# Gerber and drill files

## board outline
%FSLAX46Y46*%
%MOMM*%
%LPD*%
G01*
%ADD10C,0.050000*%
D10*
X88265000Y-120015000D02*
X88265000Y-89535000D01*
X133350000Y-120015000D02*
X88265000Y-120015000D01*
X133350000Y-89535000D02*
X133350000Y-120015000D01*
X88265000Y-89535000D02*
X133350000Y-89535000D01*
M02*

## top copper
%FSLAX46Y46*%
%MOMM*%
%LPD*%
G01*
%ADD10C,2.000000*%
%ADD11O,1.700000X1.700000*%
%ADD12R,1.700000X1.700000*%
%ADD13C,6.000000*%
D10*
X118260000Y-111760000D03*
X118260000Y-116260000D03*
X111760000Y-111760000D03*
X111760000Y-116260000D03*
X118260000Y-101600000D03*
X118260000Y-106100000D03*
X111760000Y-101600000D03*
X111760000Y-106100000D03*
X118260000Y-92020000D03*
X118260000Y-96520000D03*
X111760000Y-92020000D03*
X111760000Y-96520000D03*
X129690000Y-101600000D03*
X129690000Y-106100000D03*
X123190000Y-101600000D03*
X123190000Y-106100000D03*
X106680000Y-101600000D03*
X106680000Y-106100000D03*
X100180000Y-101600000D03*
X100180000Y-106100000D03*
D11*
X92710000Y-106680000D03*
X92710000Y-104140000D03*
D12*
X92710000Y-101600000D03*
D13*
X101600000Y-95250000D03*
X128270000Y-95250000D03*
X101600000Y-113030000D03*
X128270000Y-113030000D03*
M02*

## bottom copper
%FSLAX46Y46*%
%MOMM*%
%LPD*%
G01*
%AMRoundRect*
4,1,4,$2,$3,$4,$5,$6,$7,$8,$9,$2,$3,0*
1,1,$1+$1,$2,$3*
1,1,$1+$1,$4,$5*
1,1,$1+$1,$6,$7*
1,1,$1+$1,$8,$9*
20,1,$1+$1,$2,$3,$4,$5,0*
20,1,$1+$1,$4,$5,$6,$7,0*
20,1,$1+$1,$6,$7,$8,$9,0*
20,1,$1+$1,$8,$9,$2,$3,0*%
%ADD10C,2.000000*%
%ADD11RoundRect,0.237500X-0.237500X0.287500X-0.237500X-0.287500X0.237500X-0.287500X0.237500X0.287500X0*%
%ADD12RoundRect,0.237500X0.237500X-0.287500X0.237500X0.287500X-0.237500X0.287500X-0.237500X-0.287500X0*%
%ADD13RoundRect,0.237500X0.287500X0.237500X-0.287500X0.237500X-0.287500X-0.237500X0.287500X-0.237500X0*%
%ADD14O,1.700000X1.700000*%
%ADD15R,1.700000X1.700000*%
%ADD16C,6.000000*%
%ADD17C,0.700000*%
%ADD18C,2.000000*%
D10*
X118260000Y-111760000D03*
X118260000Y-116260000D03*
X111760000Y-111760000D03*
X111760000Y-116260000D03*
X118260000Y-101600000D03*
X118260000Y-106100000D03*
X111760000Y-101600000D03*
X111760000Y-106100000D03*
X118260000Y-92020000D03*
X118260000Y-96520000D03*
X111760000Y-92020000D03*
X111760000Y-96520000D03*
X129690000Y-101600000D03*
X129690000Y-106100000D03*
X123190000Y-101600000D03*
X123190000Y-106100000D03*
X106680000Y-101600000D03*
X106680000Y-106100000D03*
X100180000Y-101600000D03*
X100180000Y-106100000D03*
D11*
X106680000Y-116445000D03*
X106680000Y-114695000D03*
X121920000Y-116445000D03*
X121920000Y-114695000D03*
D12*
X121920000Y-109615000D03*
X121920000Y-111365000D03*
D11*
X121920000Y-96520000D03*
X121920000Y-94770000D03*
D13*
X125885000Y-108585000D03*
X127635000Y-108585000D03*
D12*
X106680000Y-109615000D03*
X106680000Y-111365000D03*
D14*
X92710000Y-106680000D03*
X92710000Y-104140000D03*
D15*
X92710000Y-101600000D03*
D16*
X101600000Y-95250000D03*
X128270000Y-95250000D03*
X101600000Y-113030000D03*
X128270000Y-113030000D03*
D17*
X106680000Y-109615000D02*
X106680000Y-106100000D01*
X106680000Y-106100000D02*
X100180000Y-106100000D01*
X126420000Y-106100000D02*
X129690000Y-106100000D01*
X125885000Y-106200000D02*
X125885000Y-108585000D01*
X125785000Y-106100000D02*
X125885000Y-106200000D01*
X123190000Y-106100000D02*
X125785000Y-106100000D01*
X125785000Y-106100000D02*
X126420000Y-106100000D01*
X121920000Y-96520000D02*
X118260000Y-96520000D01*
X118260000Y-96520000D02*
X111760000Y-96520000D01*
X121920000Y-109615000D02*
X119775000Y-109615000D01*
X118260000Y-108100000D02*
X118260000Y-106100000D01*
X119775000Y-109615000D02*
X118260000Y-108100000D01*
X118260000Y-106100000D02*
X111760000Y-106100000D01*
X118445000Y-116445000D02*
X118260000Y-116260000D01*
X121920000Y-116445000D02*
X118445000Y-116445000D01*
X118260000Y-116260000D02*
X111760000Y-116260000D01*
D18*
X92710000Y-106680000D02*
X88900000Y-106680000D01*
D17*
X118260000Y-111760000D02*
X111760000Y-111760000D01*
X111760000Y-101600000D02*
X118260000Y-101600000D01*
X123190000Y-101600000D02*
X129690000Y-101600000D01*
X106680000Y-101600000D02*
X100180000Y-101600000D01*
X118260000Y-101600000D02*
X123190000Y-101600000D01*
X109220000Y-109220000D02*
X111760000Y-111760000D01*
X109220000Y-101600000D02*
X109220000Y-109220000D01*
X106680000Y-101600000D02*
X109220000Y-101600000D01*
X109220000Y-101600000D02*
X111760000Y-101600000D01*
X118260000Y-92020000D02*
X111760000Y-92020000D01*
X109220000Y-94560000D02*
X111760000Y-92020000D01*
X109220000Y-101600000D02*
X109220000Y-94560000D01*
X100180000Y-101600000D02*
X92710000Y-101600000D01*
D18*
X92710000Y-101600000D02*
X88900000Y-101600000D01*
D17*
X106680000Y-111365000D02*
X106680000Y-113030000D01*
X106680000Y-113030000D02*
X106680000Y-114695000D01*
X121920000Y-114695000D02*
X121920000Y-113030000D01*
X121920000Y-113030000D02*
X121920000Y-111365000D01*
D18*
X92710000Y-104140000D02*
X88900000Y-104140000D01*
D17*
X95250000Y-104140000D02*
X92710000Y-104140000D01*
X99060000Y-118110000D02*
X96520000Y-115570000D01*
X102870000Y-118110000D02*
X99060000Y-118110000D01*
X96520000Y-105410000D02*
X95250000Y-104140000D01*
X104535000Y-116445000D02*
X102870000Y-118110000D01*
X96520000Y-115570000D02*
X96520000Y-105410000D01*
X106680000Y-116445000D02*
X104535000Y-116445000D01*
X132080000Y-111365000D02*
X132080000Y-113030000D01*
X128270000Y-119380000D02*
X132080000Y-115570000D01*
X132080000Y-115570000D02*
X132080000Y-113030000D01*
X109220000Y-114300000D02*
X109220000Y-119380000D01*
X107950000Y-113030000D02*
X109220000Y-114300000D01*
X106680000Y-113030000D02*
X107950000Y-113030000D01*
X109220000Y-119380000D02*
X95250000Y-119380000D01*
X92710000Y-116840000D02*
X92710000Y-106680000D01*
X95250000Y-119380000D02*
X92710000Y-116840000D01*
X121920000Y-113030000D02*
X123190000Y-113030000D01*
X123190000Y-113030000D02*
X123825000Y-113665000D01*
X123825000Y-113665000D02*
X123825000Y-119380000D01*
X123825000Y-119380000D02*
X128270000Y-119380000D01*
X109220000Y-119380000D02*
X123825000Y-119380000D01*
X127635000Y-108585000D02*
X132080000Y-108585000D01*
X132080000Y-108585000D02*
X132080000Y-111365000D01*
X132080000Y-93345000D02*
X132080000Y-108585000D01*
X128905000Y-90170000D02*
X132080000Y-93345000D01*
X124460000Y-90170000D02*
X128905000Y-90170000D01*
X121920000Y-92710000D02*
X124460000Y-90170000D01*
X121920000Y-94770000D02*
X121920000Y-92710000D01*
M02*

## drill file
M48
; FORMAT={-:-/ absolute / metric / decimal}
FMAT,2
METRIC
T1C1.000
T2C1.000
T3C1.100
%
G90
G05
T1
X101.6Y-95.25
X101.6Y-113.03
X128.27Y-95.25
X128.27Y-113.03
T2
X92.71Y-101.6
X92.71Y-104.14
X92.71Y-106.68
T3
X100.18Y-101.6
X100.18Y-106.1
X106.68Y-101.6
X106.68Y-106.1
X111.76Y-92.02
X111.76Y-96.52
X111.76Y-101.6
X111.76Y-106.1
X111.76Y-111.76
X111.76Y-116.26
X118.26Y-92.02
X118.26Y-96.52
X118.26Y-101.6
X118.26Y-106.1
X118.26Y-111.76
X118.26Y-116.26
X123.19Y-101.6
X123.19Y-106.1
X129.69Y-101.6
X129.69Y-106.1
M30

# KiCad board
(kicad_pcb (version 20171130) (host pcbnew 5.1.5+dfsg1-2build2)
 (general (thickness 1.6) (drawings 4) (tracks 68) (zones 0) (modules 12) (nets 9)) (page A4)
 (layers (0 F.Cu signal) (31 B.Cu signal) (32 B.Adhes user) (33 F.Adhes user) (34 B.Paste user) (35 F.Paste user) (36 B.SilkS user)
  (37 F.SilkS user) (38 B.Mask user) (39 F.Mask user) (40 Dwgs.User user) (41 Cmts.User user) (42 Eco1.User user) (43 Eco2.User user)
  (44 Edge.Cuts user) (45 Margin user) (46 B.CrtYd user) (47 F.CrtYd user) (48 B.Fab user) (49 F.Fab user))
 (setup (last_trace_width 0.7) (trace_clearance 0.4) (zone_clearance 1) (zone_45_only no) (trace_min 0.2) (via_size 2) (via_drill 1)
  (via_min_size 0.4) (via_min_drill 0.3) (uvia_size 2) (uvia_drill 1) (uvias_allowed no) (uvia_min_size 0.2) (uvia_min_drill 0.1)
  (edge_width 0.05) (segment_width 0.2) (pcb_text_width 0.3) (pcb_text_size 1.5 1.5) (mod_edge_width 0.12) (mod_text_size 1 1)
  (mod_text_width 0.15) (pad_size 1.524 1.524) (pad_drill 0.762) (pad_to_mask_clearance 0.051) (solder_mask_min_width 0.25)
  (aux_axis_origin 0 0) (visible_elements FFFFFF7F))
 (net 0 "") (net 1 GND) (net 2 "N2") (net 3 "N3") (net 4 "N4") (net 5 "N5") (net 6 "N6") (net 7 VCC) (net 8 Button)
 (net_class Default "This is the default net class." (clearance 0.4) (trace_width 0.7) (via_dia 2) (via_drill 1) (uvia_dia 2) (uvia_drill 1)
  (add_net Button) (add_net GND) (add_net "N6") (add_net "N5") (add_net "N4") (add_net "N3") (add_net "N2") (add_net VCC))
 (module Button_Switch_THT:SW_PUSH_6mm (layer F.Cu) (at 111.76 111.76)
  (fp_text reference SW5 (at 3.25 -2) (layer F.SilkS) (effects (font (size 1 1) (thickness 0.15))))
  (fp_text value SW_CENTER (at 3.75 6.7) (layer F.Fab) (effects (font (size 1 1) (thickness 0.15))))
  (pad 1 thru_hole circle (at 6.5 0 90) (size 2 2) (drill 1.1) (layers *.Cu *.Mask) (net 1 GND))
  (pad 2 thru_hole circle (at 6.5 4.5 90) (size 2 2) (drill 1.1) (layers *.Cu *.Mask) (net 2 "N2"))
  (pad 1 thru_hole circle (at 0 0 90) (size 2 2) (drill 1.1) (layers *.Cu *.Mask) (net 1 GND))
  (pad 2 thru_hole circle (at 0 4.5 90) (size 2 2) (drill 1.1) (layers *.Cu *.Mask) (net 2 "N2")))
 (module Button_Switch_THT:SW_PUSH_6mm (layer F.Cu) (at 111.76 101.6)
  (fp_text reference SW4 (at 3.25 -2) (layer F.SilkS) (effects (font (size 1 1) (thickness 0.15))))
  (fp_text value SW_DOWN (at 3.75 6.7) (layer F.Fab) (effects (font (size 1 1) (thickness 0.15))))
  (pad 1 thru_hole circle (at 6.5 0 90) (size 2 2) (drill 1.1) (layers *.Cu *.Mask) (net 1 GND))
  (pad 2 thru_hole circle (at 6.5 4.5 90) (size 2 2) (drill 1.1) (layers *.Cu *.Mask) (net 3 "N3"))
  (pad 1 thru_hole circle (at 0 0 90) (size 2 2) (drill 1.1) (layers *.Cu *.Mask) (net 1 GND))
  (pad 2 thru_hole circle (at 0 4.5 90) (size 2 2) (drill 1.1) (layers *.Cu *.Mask) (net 3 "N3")))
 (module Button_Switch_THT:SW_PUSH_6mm (layer F.Cu) (at 111.76 92.02)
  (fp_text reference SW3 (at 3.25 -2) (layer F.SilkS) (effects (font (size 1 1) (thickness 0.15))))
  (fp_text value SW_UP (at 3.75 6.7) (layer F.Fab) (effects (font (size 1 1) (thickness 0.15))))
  (pad 1 thru_hole circle (at 6.5 0 90) (size 2 2) (drill 1.1) (layers *.Cu *.Mask) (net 1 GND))
  (pad 2 thru_hole circle (at 6.5 4.5 90) (size 2 2) (drill 1.1) (layers *.Cu *.Mask) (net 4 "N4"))
  (pad 1 thru_hole circle (at 0 0 90) (size 2 2) (drill 1.1) (layers *.Cu *.Mask) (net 1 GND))
  (pad 2 thru_hole circle (at 0 4.5 90) (size 2 2) (drill 1.1) (layers *.Cu *.Mask) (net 4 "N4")))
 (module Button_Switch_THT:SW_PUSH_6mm (layer F.Cu) (at 123.19 101.6)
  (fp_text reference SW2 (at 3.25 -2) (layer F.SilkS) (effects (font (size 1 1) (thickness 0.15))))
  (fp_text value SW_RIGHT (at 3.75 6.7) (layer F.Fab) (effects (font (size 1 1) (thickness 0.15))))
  (pad 1 thru_hole circle (at 6.5 0 90) (size 2 2) (drill 1.1) (layers *.Cu *.Mask) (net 1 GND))
  (pad 2 thru_hole circle (at 6.5 4.5 90) (size 2 2) (drill 1.1) (layers *.Cu *.Mask) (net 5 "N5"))
  (pad 1 thru_hole circle (at 0 0 90) (size 2 2) (drill 1.1) (layers *.Cu *.Mask) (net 1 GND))
  (pad 2 thru_hole circle (at 0 4.5 90) (size 2 2) (drill 1.1) (layers *.Cu *.Mask) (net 5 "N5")))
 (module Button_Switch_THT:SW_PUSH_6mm (layer F.Cu) (at 100.18 101.6)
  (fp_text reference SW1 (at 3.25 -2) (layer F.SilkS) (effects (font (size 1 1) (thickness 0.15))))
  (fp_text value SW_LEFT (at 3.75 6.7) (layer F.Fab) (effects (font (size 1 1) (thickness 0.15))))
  (pad 1 thru_hole circle (at 6.5 0 90) (size 2 2) (drill 1.1) (layers *.Cu *.Mask) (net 1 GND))
  (pad 2 thru_hole circle (at 6.5 4.5 90) (size 2 2) (drill 1.1) (layers *.Cu *.Mask) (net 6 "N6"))
  (pad 1 thru_hole circle (at 0 0 90) (size 2 2) (drill 1.1) (layers *.Cu *.Mask) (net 1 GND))
  (pad 2 thru_hole circle (at 0 4.5 90) (size 2 2) (drill 1.1) (layers *.Cu *.Mask) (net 6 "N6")))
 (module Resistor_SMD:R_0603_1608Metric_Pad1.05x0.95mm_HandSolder (layer B.Cu) (at 106.68 115.57 270)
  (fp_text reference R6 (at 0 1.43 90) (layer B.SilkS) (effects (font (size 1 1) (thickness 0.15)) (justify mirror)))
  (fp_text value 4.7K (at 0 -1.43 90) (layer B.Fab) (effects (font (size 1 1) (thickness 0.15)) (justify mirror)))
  (pad 2 smd roundrect (at 0.875 0 270) (size 1.05 0.95) (layers B.Cu B.Paste B.Mask) (roundrect_rratio 0.25) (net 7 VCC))
  (pad 1 smd roundrect (at -0.875 0 270) (size 1.05 0.95) (layers B.Cu B.Paste B.Mask) (roundrect_rratio 0.25) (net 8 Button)))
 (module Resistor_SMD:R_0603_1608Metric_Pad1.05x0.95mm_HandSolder (layer B.Cu) (at 121.92 115.57 270)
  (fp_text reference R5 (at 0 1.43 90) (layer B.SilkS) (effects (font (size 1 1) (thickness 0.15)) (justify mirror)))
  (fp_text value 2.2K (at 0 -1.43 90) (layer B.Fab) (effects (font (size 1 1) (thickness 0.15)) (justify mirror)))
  (pad 2 smd roundrect (at 0.875 0 270) (size 1.05 0.95) (layers B.Cu B.Paste B.Mask) (roundrect_rratio 0.25) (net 2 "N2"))
  (pad 1 smd roundrect (at -0.875 0 270) (size 1.05 0.95) (layers B.Cu B.Paste B.Mask) (roundrect_rratio 0.25) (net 8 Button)))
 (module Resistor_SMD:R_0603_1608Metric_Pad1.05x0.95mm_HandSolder (layer B.Cu) (at 121.92 110.49 90)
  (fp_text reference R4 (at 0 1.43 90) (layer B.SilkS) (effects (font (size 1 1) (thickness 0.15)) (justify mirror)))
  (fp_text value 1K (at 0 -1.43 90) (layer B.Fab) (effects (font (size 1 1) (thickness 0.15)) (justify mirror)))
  (pad 2 smd roundrect (at 0.875 0 90) (size 1.05 0.95) (layers B.Cu B.Paste B.Mask) (roundrect_rratio 0.25) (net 3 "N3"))
  (pad 1 smd roundrect (at -0.875 0 90) (size 1.05 0.95) (layers B.Cu B.Paste B.Mask) (roundrect_rratio 0.25) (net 8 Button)))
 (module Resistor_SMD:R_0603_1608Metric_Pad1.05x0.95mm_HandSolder (layer B.Cu) (at 121.92 95.645 270)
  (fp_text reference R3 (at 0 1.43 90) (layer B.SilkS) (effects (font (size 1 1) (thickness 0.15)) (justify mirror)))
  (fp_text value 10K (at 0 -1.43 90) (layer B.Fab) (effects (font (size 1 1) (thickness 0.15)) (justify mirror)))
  (pad 2 smd roundrect (at 0.875 0 270) (size 1.05 0.95) (layers B.Cu B.Paste B.Mask) (roundrect_rratio 0.25) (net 4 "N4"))
  (pad 1 smd roundrect (at -0.875 0 270) (size 1.05 0.95) (layers B.Cu B.Paste B.Mask) (roundrect_rratio 0.25) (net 8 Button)))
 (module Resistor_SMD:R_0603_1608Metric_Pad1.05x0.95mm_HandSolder (layer B.Cu) (at 126.76 108.585 180)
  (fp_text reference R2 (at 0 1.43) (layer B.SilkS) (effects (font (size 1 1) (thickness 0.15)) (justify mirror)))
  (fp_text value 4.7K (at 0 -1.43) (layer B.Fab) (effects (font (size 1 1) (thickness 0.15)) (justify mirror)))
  (pad 2 smd roundrect (at 0.875 0 180) (size 1.05 0.95) (layers B.Cu B.Paste B.Mask) (roundrect_rratio 0.25) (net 5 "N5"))
  (pad 1 smd roundrect (at -0.875 0 180) (size 1.05 0.95) (layers B.Cu B.Paste B.Mask) (roundrect_rratio 0.25) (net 8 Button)))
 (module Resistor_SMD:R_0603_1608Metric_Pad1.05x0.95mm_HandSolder (layer B.Cu) (at 106.68 110.49 90)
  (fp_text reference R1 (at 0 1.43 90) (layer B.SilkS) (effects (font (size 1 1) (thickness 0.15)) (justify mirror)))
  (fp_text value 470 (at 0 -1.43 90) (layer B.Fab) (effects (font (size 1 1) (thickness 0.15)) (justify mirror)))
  (pad 2 smd roundrect (at 0.875 0 90) (size 1.05 0.95) (layers B.Cu B.Paste B.Mask) (roundrect_rratio 0.25) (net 6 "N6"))
  (pad 1 smd roundrect (at -0.875 0 90) (size 1.05 0.95) (layers B.Cu B.Paste B.Mask) (roundrect_rratio 0.25) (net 8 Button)))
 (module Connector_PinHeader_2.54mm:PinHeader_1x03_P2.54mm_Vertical (layer F.Cu) (at 92.71 101.6)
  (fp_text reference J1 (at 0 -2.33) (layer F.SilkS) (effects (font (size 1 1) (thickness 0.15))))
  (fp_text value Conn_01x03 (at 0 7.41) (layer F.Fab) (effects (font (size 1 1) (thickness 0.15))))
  (pad 3 thru_hole oval (at 0 5.08) (size 1.7 1.7) (drill 1) (layers *.Cu *.Mask) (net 8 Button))
  (pad 2 thru_hole oval (at 0 2.54) (size 1.7 1.7) (drill 1) (layers *.Cu *.Mask) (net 7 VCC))
  (pad 1 thru_hole rect (at 0 0) (size 1.7 1.7) (drill 1) (layers *.Cu *.Mask) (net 1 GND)))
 (gr_line (start 88.265 120.015) (end 88.265 89.535) (layer Edge.Cuts) (width 0.05))
 (gr_line (start 133.35 120.015) (end 88.265 120.015) (layer Edge.Cuts) (width 0.05))
 (gr_line (start 133.35 89.535) (end 133.35 120.015) (layer Edge.Cuts) (width 0.05))
 (gr_line (start 88.265 89.535) (end 133.35 89.535) (layer Edge.Cuts) (width 0.05))
 (via (at 101.6 95.25) (size 6) (drill 1) (layers F.Cu B.Cu) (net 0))
 (via (at 128.27 95.25) (size 6) (drill 1) (layers F.Cu B.Cu) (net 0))
 (via (at 101.6 113.03) (size 6) (drill 1) (layers F.Cu B.Cu) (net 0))
 (via (at 128.27 113.03) (size 6) (drill 1) (layers F.Cu B.Cu) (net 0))
 (segment (start 106.68 109.615) (end 106.68 106.1) (width 0.7) (layer B.Cu) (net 6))
 (segment (start 106.68 106.1) (end 100.18 106.1) (width 0.7) (layer B.Cu) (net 6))
 (segment (start 126.42 106.1) (end 129.69 106.1) (width 0.7) (layer B.Cu) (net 5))
 (segment (start 125.885 106.2) (end 125.885 108.585) (width 0.7) (layer B.Cu) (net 5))
 (segment (start 125.785 106.1) (end 125.885 106.2) (width 0.7) (layer B.Cu) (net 5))
 (segment (start 123.19 106.1) (end 125.785 106.1) (width 0.7) (layer B.Cu) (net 5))
 (segment (start 125.785 106.1) (end 126.42 106.1) (width 0.7) (layer B.Cu) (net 5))
 (segment (start 121.92 96.52) (end 118.26 96.52) (width 0.7) (layer B.Cu) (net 4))
 (segment (start 118.26 96.52) (end 111.76 96.52) (width 0.7) (layer B.Cu) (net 4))
 (segment (start 121.92 109.615) (end 119.775 109.615) (width 0.7) (layer B.Cu) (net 3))
 (segment (start 118.26 108.1) (end 118.26 106.1) (width 0.7) (layer B.Cu) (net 3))
 (segment (start 119.775 109.615) (end 118.26 108.1) (width 0.7) (layer B.Cu) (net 3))
 (segment (start 118.26 106.1) (end 111.76 106.1) (width 0.7) (layer B.Cu) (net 3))
 (segment (start 118.445 116.445) (end 118.26 116.26) (width 0.7) (layer B.Cu) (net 2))
 (segment (start 121.92 116.445) (end 118.445 116.445) (width 0.7) (layer B.Cu) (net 2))
 (segment (start 118.26 116.26) (end 111.76 116.26) (width 0.7) (layer B.Cu) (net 2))
 (segment (start 92.71 106.68) (end 88.9 106.68) (width 2) (layer B.Cu) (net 8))
 (segment (start 118.26 111.76) (end 111.76 111.76) (width 0.7) (layer B.Cu) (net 1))
 (segment (start 111.76 101.6) (end 118.26 101.6) (width 0.7) (layer B.Cu) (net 1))
 (segment (start 123.19 101.6) (end 129.69 101.6) (width 0.7) (layer B.Cu) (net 1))
 (segment (start 106.68 101.6) (end 100.18 101.6) (width 0.7) (layer B.Cu) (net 1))
 (segment (start 118.26 101.6) (end 123.19 101.6) (width 0.7) (layer B.Cu) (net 1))
 (segment (start 109.22 109.22) (end 111.76 111.76) (width 0.7) (layer B.Cu) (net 1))
 (segment (start 109.22 101.6) (end 109.22 109.22) (width 0.7) (layer B.Cu) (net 1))
 (segment (start 106.68 101.6) (end 109.22 101.6) (width 0.7) (layer B.Cu) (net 1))
 (segment (start 109.22 101.6) (end 111.76 101.6) (width 0.7) (layer B.Cu) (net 1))
 (segment (start 118.26 92.02) (end 111.76 92.02) (width 0.7) (layer B.Cu) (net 1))
 (segment (start 109.22 94.56) (end 111.76 92.02) (width 0.7) (layer B.Cu) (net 1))
 (segment (start 109.22 101.6) (end 109.22 94.56) (width 0.7) (layer B.Cu) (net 1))
 (segment (start 100.18 101.6) (end 92.71 101.6) (width 0.7) (layer B.Cu) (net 1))
 (segment (start 92.71 101.6) (end 88.9 101.6) (width 2) (layer B.Cu) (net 1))
 (segment (start 106.68 111.365) (end 106.68 113.03) (width 0.7) (layer B.Cu) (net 8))
 (segment (start 106.68 113.03) (end 106.68 114.695) (width 0.7) (layer B.Cu) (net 8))
 (segment (start 121.92 114.695) (end 121.92 113.03) (width 0.7) (layer B.Cu) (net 8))
 (segment (start 121.92 113.03) (end 121.92 111.365) (width 0.7) (layer B.Cu) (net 8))
 (segment (start 92.71 104.14) (end 88.9 104.14) (width 2) (layer B.Cu) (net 7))
 (segment (start 95.25 104.14) (end 92.71 104.14) (width 0.7) (layer B.Cu) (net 7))
 (segment (start 99.06 118.11) (end 96.52 115.57) (width 0.7) (layer B.Cu) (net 7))
 (segment (start 102.87 118.11) (end 99.06 118.11) (width 0.7) (layer B.Cu) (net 7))
 (segment (start 96.52 105.41) (end 95.25 104.14) (width 0.7) (layer B.Cu) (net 7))
 (segment (start 104.535 116.445) (end 102.87 118.11) (width 0.7) (layer B.Cu) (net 7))
 (segment (start 96.52 115.57) (end 96.52 105.41) (width 0.7) (layer B.Cu) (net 7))
 (segment (start 106.68 116.445) (end 104.535 116.445) (width 0.7) (layer B.Cu) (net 7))
 (segment (start 132.08 111.365) (end 132.08 113.03) (width 0.7) (layer B.Cu) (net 8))
 (segment (start 128.27 119.38) (end 132.08 115.57) (width 0.7) (layer B.Cu) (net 8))
 (segment (start 132.08 115.57) (end 132.08 113.03) (width 0.7) (layer B.Cu) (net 8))
 (segment (start 109.22 114.3) (end 109.22 119.38) (width 0.7) (layer B.Cu) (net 8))
 (segment (start 107.95 113.03) (end 109.22 114.3) (width 0.7) (layer B.Cu) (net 8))
 (segment (start 106.68 113.03) (end 107.95 113.03) (width 0.7) (layer B.Cu) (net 8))
 (segment (start 109.22 119.38) (end 95.25 119.38) (width 0.7) (layer B.Cu) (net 8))
 (segment (start 92.71 116.84) (end 92.71 106.68) (width 0.7) (layer B.Cu) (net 8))
 (segment (start 95.25 119.38) (end 92.71 116.84) (width 0.7) (layer B.Cu) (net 8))
 (segment (start 121.92 113.03) (end 123.19 113.03) (width 0.7) (layer B.Cu) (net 8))
 (segment (start 123.19 113.03) (end 123.825 113.665) (width 0.7) (layer B.Cu) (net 8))
 (segment (start 123.825 113.665) (end 123.825 119.38) (width 0.7) (layer B.Cu) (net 8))
 (segment (start 123.825 119.38) (end 128.27 119.38) (width 0.7) (layer B.Cu) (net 8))
 (segment (start 109.22 119.38) (end 123.825 119.38) (width 0.7) (layer B.Cu) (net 8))
 (segment (start 127.635 108.585) (end 132.08 108.585) (width 0.7) (layer B.Cu) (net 8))
 (segment (start 132.08 108.585) (end 132.08 111.365) (width 0.7) (layer B.Cu) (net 8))
 (segment (start 132.08 93.345) (end 132.08 108.585) (width 0.7) (layer B.Cu) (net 8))
 (segment (start 128.905 90.17) (end 132.08 93.345) (width 0.7) (layer B.Cu) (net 8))
 (segment (start 124.46 90.17) (end 128.905 90.17) (width 0.7) (layer B.Cu) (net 8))
 (segment (start 121.92 92.71) (end 124.46 90.17) (width 0.7) (layer B.Cu) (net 8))
 (segment (start 121.92 94.77) (end 121.92 92.71) (width 0.7) (layer B.Cu) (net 8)))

